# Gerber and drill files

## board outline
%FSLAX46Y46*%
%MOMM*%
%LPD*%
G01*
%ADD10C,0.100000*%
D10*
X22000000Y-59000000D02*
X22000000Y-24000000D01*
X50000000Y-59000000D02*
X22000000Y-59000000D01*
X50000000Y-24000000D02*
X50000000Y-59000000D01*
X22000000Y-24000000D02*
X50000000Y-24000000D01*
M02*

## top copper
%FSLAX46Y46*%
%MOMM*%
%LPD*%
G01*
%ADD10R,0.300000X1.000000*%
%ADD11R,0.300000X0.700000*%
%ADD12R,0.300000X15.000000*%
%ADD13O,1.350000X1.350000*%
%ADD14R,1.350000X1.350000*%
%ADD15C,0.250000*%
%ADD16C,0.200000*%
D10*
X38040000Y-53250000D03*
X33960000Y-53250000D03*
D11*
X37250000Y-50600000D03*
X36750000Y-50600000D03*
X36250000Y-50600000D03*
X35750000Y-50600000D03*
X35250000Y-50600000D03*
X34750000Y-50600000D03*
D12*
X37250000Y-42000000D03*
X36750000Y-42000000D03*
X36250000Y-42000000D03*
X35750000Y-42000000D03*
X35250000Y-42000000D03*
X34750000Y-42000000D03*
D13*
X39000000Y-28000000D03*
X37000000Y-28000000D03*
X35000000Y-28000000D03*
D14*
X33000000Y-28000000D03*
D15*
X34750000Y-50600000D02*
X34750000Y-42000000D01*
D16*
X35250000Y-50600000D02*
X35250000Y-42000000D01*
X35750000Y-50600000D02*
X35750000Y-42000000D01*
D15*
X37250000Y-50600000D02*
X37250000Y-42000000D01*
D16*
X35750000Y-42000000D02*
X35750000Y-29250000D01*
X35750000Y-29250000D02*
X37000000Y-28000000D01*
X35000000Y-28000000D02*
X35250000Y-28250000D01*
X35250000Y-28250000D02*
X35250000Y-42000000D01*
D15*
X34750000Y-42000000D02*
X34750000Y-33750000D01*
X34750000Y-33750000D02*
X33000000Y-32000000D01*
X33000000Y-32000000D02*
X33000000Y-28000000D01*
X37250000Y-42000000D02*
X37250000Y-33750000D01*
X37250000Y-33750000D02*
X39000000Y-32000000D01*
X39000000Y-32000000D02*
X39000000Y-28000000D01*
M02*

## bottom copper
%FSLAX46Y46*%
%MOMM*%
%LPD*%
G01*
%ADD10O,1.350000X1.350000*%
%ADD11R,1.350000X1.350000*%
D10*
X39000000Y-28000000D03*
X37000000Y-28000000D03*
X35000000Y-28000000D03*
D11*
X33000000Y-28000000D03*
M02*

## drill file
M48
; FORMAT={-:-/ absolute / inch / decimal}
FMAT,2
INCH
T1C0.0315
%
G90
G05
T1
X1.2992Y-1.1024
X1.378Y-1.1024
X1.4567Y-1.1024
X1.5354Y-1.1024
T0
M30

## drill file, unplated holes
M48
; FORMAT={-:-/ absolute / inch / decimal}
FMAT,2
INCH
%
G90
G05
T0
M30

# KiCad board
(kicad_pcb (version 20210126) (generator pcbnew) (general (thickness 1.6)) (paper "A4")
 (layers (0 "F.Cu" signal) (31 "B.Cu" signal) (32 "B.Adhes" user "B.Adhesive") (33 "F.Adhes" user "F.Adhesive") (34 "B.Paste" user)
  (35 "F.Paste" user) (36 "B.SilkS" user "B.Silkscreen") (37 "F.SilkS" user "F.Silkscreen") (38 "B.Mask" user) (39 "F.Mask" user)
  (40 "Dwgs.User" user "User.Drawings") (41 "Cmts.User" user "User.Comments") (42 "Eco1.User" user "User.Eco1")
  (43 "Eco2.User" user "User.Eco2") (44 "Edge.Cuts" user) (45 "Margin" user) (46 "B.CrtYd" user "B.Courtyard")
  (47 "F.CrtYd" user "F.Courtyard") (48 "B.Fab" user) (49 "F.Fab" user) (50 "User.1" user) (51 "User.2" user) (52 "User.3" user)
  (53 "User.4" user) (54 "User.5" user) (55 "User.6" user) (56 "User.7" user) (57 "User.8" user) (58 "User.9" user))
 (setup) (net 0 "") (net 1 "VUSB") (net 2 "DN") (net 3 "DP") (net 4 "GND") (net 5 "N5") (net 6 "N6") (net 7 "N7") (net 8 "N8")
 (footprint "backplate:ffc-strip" (layer "F.Cu") (at 36 42)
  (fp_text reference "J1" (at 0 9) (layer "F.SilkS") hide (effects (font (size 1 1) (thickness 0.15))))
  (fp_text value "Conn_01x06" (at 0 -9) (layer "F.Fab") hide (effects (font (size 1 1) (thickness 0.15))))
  (pad "1" smd rect (at -1.25 0) (locked) (size 0.3 15) (layers "F.Cu" "F.Paste" "F.Mask") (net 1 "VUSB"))
  (pad "2" smd rect (at -0.75 0) (locked) (size 0.3 15) (layers "F.Cu" "F.Paste" "F.Mask") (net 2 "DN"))
  (pad "3" smd rect (at -0.25 0) (locked) (size 0.3 15) (layers "F.Cu" "F.Paste" "F.Mask") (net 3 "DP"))
  (pad "4" smd rect (at 0.25 0) (locked) (size 0.3 15) (layers "F.Cu" "F.Paste" "F.Mask"))
  (pad "5" smd rect (at 0.75 0) (locked) (size 0.3 15) (layers "F.Cu" "F.Paste" "F.Mask"))
  (pad "6" smd rect (at 1.25 0) (locked) (size 0.3 15) (layers "F.Cu" "F.Paste" "F.Mask") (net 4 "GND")))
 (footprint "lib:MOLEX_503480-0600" (layer "F.Cu") (at 36 52)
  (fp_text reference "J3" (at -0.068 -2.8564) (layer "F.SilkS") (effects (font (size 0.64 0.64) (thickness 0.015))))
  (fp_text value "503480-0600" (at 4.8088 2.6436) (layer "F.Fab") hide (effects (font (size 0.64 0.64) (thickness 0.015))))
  (pad "1" smd rect (at -1.25 -1.4) (locked) (size 0.3 0.7) (layers "F.Cu" "F.Paste" "F.Mask") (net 1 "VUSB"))
  (pad "2" smd rect (at -0.75 -1.4) (locked) (size 0.3 0.7) (layers "F.Cu" "F.Paste" "F.Mask") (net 2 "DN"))
  (pad "3" smd rect (at -0.25 -1.4) (locked) (size 0.3 0.7) (layers "F.Cu" "F.Paste" "F.Mask") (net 3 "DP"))
  (pad "4" smd rect (at 0.25 -1.4) (locked) (size 0.3 0.7) (layers "F.Cu" "F.Paste" "F.Mask") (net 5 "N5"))
  (pad "5" smd rect (at 0.75 -1.4) (locked) (size 0.3 0.7) (layers "F.Cu" "F.Paste" "F.Mask") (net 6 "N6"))
  (pad "6" smd rect (at 1.25 -1.4) (locked) (size 0.3 0.7) (layers "F.Cu" "F.Paste" "F.Mask") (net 4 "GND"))
  (pad "S1" smd rect (at -2.04 1.25) (locked) (size 0.3 1) (layers "F.Cu" "F.Paste" "F.Mask") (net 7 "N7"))
  (pad "S2" smd rect (at 2.04 1.25) (locked) (size 0.3 1) (layers "F.Cu" "F.Paste" "F.Mask") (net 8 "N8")))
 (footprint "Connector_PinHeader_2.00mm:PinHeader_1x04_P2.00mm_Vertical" (layer "F.Cu") (at 33 28 90)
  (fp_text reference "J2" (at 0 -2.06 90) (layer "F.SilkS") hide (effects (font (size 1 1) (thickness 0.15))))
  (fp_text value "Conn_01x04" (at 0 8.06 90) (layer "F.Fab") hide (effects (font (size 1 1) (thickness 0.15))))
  (pad "1" thru_hole rect (at 0 0 90) (locked) (size 1.35 1.35) (drill 0.8) (layers *.Cu *.Mask) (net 1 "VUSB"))
  (pad "2" thru_hole oval (at 0 2 90) (locked) (size 1.35 1.35) (drill 0.8) (layers *.Cu *.Mask) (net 2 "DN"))
  (pad "3" thru_hole oval (at 0 4 90) (locked) (size 1.35 1.35) (drill 0.8) (layers *.Cu *.Mask) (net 3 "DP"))
  (pad "4" thru_hole oval (at 0 6 90) (locked) (size 1.35 1.35) (drill 0.8) (layers *.Cu *.Mask) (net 4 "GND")))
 (gr_line (start 50 59) (end 22 59) (layer "Edge.Cuts") (width 0.1))
 (gr_line (start 22 59) (end 22 24) (layer "Edge.Cuts") (width 0.1))
 (gr_line (start 22 24) (end 50 24) (layer "Edge.Cuts") (width 0.1))
 (gr_line (start 50 24) (end 50 59) (layer "Edge.Cuts") (width 0.1))
 (segment (start 37.25 42) (end 37.25 33.75) (width 0.25) (layer "F.Cu") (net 4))
 (segment (start 39 32) (end 39 28) (width 0.25) (layer "F.Cu") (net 4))
 (segment (start 37.25 50.6) (end 37.25 42) (width 0.25) (layer "F.Cu") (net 4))
 (segment (start 37.25 33.75) (end 39 32) (width 0.25) (layer "F.Cu") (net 4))
 (segment (start 35.75 29.25) (end 37 28) (width 0.2) (layer "F.Cu") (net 3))
 (segment (start 35.75 42) (end 35.75 29.25) (width 0.2) (layer "F.Cu") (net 3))
 (segment (start 35.75 50.6) (end 35.75 42) (width 0.2) (layer "F.Cu") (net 3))
 (segment (start 35 28) (end 35.25 28.25) (width 0.2) (layer "F.Cu") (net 2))
 (segment (start 35.25 28.25) (end 35.25 42) (width 0.2) (layer "F.Cu") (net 2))
 (segment (start 35.25 50.6) (end 35.25 42) (width 0.2) (layer "F.Cu") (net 2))
 (segment (start 34.75 50.6) (end 34.75 42) (width 0.25) (layer "F.Cu") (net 1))
 (segment (start 34.75 33.75) (end 33 32) (width 0.25) (layer "F.Cu") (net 1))
 (segment (start 33 32) (end 33 28) (width 0.25) (layer "F.Cu") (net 1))
 (segment (start 34.75 42) (end 34.75 33.75) (width 0.25) (layer "F.Cu") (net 1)))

